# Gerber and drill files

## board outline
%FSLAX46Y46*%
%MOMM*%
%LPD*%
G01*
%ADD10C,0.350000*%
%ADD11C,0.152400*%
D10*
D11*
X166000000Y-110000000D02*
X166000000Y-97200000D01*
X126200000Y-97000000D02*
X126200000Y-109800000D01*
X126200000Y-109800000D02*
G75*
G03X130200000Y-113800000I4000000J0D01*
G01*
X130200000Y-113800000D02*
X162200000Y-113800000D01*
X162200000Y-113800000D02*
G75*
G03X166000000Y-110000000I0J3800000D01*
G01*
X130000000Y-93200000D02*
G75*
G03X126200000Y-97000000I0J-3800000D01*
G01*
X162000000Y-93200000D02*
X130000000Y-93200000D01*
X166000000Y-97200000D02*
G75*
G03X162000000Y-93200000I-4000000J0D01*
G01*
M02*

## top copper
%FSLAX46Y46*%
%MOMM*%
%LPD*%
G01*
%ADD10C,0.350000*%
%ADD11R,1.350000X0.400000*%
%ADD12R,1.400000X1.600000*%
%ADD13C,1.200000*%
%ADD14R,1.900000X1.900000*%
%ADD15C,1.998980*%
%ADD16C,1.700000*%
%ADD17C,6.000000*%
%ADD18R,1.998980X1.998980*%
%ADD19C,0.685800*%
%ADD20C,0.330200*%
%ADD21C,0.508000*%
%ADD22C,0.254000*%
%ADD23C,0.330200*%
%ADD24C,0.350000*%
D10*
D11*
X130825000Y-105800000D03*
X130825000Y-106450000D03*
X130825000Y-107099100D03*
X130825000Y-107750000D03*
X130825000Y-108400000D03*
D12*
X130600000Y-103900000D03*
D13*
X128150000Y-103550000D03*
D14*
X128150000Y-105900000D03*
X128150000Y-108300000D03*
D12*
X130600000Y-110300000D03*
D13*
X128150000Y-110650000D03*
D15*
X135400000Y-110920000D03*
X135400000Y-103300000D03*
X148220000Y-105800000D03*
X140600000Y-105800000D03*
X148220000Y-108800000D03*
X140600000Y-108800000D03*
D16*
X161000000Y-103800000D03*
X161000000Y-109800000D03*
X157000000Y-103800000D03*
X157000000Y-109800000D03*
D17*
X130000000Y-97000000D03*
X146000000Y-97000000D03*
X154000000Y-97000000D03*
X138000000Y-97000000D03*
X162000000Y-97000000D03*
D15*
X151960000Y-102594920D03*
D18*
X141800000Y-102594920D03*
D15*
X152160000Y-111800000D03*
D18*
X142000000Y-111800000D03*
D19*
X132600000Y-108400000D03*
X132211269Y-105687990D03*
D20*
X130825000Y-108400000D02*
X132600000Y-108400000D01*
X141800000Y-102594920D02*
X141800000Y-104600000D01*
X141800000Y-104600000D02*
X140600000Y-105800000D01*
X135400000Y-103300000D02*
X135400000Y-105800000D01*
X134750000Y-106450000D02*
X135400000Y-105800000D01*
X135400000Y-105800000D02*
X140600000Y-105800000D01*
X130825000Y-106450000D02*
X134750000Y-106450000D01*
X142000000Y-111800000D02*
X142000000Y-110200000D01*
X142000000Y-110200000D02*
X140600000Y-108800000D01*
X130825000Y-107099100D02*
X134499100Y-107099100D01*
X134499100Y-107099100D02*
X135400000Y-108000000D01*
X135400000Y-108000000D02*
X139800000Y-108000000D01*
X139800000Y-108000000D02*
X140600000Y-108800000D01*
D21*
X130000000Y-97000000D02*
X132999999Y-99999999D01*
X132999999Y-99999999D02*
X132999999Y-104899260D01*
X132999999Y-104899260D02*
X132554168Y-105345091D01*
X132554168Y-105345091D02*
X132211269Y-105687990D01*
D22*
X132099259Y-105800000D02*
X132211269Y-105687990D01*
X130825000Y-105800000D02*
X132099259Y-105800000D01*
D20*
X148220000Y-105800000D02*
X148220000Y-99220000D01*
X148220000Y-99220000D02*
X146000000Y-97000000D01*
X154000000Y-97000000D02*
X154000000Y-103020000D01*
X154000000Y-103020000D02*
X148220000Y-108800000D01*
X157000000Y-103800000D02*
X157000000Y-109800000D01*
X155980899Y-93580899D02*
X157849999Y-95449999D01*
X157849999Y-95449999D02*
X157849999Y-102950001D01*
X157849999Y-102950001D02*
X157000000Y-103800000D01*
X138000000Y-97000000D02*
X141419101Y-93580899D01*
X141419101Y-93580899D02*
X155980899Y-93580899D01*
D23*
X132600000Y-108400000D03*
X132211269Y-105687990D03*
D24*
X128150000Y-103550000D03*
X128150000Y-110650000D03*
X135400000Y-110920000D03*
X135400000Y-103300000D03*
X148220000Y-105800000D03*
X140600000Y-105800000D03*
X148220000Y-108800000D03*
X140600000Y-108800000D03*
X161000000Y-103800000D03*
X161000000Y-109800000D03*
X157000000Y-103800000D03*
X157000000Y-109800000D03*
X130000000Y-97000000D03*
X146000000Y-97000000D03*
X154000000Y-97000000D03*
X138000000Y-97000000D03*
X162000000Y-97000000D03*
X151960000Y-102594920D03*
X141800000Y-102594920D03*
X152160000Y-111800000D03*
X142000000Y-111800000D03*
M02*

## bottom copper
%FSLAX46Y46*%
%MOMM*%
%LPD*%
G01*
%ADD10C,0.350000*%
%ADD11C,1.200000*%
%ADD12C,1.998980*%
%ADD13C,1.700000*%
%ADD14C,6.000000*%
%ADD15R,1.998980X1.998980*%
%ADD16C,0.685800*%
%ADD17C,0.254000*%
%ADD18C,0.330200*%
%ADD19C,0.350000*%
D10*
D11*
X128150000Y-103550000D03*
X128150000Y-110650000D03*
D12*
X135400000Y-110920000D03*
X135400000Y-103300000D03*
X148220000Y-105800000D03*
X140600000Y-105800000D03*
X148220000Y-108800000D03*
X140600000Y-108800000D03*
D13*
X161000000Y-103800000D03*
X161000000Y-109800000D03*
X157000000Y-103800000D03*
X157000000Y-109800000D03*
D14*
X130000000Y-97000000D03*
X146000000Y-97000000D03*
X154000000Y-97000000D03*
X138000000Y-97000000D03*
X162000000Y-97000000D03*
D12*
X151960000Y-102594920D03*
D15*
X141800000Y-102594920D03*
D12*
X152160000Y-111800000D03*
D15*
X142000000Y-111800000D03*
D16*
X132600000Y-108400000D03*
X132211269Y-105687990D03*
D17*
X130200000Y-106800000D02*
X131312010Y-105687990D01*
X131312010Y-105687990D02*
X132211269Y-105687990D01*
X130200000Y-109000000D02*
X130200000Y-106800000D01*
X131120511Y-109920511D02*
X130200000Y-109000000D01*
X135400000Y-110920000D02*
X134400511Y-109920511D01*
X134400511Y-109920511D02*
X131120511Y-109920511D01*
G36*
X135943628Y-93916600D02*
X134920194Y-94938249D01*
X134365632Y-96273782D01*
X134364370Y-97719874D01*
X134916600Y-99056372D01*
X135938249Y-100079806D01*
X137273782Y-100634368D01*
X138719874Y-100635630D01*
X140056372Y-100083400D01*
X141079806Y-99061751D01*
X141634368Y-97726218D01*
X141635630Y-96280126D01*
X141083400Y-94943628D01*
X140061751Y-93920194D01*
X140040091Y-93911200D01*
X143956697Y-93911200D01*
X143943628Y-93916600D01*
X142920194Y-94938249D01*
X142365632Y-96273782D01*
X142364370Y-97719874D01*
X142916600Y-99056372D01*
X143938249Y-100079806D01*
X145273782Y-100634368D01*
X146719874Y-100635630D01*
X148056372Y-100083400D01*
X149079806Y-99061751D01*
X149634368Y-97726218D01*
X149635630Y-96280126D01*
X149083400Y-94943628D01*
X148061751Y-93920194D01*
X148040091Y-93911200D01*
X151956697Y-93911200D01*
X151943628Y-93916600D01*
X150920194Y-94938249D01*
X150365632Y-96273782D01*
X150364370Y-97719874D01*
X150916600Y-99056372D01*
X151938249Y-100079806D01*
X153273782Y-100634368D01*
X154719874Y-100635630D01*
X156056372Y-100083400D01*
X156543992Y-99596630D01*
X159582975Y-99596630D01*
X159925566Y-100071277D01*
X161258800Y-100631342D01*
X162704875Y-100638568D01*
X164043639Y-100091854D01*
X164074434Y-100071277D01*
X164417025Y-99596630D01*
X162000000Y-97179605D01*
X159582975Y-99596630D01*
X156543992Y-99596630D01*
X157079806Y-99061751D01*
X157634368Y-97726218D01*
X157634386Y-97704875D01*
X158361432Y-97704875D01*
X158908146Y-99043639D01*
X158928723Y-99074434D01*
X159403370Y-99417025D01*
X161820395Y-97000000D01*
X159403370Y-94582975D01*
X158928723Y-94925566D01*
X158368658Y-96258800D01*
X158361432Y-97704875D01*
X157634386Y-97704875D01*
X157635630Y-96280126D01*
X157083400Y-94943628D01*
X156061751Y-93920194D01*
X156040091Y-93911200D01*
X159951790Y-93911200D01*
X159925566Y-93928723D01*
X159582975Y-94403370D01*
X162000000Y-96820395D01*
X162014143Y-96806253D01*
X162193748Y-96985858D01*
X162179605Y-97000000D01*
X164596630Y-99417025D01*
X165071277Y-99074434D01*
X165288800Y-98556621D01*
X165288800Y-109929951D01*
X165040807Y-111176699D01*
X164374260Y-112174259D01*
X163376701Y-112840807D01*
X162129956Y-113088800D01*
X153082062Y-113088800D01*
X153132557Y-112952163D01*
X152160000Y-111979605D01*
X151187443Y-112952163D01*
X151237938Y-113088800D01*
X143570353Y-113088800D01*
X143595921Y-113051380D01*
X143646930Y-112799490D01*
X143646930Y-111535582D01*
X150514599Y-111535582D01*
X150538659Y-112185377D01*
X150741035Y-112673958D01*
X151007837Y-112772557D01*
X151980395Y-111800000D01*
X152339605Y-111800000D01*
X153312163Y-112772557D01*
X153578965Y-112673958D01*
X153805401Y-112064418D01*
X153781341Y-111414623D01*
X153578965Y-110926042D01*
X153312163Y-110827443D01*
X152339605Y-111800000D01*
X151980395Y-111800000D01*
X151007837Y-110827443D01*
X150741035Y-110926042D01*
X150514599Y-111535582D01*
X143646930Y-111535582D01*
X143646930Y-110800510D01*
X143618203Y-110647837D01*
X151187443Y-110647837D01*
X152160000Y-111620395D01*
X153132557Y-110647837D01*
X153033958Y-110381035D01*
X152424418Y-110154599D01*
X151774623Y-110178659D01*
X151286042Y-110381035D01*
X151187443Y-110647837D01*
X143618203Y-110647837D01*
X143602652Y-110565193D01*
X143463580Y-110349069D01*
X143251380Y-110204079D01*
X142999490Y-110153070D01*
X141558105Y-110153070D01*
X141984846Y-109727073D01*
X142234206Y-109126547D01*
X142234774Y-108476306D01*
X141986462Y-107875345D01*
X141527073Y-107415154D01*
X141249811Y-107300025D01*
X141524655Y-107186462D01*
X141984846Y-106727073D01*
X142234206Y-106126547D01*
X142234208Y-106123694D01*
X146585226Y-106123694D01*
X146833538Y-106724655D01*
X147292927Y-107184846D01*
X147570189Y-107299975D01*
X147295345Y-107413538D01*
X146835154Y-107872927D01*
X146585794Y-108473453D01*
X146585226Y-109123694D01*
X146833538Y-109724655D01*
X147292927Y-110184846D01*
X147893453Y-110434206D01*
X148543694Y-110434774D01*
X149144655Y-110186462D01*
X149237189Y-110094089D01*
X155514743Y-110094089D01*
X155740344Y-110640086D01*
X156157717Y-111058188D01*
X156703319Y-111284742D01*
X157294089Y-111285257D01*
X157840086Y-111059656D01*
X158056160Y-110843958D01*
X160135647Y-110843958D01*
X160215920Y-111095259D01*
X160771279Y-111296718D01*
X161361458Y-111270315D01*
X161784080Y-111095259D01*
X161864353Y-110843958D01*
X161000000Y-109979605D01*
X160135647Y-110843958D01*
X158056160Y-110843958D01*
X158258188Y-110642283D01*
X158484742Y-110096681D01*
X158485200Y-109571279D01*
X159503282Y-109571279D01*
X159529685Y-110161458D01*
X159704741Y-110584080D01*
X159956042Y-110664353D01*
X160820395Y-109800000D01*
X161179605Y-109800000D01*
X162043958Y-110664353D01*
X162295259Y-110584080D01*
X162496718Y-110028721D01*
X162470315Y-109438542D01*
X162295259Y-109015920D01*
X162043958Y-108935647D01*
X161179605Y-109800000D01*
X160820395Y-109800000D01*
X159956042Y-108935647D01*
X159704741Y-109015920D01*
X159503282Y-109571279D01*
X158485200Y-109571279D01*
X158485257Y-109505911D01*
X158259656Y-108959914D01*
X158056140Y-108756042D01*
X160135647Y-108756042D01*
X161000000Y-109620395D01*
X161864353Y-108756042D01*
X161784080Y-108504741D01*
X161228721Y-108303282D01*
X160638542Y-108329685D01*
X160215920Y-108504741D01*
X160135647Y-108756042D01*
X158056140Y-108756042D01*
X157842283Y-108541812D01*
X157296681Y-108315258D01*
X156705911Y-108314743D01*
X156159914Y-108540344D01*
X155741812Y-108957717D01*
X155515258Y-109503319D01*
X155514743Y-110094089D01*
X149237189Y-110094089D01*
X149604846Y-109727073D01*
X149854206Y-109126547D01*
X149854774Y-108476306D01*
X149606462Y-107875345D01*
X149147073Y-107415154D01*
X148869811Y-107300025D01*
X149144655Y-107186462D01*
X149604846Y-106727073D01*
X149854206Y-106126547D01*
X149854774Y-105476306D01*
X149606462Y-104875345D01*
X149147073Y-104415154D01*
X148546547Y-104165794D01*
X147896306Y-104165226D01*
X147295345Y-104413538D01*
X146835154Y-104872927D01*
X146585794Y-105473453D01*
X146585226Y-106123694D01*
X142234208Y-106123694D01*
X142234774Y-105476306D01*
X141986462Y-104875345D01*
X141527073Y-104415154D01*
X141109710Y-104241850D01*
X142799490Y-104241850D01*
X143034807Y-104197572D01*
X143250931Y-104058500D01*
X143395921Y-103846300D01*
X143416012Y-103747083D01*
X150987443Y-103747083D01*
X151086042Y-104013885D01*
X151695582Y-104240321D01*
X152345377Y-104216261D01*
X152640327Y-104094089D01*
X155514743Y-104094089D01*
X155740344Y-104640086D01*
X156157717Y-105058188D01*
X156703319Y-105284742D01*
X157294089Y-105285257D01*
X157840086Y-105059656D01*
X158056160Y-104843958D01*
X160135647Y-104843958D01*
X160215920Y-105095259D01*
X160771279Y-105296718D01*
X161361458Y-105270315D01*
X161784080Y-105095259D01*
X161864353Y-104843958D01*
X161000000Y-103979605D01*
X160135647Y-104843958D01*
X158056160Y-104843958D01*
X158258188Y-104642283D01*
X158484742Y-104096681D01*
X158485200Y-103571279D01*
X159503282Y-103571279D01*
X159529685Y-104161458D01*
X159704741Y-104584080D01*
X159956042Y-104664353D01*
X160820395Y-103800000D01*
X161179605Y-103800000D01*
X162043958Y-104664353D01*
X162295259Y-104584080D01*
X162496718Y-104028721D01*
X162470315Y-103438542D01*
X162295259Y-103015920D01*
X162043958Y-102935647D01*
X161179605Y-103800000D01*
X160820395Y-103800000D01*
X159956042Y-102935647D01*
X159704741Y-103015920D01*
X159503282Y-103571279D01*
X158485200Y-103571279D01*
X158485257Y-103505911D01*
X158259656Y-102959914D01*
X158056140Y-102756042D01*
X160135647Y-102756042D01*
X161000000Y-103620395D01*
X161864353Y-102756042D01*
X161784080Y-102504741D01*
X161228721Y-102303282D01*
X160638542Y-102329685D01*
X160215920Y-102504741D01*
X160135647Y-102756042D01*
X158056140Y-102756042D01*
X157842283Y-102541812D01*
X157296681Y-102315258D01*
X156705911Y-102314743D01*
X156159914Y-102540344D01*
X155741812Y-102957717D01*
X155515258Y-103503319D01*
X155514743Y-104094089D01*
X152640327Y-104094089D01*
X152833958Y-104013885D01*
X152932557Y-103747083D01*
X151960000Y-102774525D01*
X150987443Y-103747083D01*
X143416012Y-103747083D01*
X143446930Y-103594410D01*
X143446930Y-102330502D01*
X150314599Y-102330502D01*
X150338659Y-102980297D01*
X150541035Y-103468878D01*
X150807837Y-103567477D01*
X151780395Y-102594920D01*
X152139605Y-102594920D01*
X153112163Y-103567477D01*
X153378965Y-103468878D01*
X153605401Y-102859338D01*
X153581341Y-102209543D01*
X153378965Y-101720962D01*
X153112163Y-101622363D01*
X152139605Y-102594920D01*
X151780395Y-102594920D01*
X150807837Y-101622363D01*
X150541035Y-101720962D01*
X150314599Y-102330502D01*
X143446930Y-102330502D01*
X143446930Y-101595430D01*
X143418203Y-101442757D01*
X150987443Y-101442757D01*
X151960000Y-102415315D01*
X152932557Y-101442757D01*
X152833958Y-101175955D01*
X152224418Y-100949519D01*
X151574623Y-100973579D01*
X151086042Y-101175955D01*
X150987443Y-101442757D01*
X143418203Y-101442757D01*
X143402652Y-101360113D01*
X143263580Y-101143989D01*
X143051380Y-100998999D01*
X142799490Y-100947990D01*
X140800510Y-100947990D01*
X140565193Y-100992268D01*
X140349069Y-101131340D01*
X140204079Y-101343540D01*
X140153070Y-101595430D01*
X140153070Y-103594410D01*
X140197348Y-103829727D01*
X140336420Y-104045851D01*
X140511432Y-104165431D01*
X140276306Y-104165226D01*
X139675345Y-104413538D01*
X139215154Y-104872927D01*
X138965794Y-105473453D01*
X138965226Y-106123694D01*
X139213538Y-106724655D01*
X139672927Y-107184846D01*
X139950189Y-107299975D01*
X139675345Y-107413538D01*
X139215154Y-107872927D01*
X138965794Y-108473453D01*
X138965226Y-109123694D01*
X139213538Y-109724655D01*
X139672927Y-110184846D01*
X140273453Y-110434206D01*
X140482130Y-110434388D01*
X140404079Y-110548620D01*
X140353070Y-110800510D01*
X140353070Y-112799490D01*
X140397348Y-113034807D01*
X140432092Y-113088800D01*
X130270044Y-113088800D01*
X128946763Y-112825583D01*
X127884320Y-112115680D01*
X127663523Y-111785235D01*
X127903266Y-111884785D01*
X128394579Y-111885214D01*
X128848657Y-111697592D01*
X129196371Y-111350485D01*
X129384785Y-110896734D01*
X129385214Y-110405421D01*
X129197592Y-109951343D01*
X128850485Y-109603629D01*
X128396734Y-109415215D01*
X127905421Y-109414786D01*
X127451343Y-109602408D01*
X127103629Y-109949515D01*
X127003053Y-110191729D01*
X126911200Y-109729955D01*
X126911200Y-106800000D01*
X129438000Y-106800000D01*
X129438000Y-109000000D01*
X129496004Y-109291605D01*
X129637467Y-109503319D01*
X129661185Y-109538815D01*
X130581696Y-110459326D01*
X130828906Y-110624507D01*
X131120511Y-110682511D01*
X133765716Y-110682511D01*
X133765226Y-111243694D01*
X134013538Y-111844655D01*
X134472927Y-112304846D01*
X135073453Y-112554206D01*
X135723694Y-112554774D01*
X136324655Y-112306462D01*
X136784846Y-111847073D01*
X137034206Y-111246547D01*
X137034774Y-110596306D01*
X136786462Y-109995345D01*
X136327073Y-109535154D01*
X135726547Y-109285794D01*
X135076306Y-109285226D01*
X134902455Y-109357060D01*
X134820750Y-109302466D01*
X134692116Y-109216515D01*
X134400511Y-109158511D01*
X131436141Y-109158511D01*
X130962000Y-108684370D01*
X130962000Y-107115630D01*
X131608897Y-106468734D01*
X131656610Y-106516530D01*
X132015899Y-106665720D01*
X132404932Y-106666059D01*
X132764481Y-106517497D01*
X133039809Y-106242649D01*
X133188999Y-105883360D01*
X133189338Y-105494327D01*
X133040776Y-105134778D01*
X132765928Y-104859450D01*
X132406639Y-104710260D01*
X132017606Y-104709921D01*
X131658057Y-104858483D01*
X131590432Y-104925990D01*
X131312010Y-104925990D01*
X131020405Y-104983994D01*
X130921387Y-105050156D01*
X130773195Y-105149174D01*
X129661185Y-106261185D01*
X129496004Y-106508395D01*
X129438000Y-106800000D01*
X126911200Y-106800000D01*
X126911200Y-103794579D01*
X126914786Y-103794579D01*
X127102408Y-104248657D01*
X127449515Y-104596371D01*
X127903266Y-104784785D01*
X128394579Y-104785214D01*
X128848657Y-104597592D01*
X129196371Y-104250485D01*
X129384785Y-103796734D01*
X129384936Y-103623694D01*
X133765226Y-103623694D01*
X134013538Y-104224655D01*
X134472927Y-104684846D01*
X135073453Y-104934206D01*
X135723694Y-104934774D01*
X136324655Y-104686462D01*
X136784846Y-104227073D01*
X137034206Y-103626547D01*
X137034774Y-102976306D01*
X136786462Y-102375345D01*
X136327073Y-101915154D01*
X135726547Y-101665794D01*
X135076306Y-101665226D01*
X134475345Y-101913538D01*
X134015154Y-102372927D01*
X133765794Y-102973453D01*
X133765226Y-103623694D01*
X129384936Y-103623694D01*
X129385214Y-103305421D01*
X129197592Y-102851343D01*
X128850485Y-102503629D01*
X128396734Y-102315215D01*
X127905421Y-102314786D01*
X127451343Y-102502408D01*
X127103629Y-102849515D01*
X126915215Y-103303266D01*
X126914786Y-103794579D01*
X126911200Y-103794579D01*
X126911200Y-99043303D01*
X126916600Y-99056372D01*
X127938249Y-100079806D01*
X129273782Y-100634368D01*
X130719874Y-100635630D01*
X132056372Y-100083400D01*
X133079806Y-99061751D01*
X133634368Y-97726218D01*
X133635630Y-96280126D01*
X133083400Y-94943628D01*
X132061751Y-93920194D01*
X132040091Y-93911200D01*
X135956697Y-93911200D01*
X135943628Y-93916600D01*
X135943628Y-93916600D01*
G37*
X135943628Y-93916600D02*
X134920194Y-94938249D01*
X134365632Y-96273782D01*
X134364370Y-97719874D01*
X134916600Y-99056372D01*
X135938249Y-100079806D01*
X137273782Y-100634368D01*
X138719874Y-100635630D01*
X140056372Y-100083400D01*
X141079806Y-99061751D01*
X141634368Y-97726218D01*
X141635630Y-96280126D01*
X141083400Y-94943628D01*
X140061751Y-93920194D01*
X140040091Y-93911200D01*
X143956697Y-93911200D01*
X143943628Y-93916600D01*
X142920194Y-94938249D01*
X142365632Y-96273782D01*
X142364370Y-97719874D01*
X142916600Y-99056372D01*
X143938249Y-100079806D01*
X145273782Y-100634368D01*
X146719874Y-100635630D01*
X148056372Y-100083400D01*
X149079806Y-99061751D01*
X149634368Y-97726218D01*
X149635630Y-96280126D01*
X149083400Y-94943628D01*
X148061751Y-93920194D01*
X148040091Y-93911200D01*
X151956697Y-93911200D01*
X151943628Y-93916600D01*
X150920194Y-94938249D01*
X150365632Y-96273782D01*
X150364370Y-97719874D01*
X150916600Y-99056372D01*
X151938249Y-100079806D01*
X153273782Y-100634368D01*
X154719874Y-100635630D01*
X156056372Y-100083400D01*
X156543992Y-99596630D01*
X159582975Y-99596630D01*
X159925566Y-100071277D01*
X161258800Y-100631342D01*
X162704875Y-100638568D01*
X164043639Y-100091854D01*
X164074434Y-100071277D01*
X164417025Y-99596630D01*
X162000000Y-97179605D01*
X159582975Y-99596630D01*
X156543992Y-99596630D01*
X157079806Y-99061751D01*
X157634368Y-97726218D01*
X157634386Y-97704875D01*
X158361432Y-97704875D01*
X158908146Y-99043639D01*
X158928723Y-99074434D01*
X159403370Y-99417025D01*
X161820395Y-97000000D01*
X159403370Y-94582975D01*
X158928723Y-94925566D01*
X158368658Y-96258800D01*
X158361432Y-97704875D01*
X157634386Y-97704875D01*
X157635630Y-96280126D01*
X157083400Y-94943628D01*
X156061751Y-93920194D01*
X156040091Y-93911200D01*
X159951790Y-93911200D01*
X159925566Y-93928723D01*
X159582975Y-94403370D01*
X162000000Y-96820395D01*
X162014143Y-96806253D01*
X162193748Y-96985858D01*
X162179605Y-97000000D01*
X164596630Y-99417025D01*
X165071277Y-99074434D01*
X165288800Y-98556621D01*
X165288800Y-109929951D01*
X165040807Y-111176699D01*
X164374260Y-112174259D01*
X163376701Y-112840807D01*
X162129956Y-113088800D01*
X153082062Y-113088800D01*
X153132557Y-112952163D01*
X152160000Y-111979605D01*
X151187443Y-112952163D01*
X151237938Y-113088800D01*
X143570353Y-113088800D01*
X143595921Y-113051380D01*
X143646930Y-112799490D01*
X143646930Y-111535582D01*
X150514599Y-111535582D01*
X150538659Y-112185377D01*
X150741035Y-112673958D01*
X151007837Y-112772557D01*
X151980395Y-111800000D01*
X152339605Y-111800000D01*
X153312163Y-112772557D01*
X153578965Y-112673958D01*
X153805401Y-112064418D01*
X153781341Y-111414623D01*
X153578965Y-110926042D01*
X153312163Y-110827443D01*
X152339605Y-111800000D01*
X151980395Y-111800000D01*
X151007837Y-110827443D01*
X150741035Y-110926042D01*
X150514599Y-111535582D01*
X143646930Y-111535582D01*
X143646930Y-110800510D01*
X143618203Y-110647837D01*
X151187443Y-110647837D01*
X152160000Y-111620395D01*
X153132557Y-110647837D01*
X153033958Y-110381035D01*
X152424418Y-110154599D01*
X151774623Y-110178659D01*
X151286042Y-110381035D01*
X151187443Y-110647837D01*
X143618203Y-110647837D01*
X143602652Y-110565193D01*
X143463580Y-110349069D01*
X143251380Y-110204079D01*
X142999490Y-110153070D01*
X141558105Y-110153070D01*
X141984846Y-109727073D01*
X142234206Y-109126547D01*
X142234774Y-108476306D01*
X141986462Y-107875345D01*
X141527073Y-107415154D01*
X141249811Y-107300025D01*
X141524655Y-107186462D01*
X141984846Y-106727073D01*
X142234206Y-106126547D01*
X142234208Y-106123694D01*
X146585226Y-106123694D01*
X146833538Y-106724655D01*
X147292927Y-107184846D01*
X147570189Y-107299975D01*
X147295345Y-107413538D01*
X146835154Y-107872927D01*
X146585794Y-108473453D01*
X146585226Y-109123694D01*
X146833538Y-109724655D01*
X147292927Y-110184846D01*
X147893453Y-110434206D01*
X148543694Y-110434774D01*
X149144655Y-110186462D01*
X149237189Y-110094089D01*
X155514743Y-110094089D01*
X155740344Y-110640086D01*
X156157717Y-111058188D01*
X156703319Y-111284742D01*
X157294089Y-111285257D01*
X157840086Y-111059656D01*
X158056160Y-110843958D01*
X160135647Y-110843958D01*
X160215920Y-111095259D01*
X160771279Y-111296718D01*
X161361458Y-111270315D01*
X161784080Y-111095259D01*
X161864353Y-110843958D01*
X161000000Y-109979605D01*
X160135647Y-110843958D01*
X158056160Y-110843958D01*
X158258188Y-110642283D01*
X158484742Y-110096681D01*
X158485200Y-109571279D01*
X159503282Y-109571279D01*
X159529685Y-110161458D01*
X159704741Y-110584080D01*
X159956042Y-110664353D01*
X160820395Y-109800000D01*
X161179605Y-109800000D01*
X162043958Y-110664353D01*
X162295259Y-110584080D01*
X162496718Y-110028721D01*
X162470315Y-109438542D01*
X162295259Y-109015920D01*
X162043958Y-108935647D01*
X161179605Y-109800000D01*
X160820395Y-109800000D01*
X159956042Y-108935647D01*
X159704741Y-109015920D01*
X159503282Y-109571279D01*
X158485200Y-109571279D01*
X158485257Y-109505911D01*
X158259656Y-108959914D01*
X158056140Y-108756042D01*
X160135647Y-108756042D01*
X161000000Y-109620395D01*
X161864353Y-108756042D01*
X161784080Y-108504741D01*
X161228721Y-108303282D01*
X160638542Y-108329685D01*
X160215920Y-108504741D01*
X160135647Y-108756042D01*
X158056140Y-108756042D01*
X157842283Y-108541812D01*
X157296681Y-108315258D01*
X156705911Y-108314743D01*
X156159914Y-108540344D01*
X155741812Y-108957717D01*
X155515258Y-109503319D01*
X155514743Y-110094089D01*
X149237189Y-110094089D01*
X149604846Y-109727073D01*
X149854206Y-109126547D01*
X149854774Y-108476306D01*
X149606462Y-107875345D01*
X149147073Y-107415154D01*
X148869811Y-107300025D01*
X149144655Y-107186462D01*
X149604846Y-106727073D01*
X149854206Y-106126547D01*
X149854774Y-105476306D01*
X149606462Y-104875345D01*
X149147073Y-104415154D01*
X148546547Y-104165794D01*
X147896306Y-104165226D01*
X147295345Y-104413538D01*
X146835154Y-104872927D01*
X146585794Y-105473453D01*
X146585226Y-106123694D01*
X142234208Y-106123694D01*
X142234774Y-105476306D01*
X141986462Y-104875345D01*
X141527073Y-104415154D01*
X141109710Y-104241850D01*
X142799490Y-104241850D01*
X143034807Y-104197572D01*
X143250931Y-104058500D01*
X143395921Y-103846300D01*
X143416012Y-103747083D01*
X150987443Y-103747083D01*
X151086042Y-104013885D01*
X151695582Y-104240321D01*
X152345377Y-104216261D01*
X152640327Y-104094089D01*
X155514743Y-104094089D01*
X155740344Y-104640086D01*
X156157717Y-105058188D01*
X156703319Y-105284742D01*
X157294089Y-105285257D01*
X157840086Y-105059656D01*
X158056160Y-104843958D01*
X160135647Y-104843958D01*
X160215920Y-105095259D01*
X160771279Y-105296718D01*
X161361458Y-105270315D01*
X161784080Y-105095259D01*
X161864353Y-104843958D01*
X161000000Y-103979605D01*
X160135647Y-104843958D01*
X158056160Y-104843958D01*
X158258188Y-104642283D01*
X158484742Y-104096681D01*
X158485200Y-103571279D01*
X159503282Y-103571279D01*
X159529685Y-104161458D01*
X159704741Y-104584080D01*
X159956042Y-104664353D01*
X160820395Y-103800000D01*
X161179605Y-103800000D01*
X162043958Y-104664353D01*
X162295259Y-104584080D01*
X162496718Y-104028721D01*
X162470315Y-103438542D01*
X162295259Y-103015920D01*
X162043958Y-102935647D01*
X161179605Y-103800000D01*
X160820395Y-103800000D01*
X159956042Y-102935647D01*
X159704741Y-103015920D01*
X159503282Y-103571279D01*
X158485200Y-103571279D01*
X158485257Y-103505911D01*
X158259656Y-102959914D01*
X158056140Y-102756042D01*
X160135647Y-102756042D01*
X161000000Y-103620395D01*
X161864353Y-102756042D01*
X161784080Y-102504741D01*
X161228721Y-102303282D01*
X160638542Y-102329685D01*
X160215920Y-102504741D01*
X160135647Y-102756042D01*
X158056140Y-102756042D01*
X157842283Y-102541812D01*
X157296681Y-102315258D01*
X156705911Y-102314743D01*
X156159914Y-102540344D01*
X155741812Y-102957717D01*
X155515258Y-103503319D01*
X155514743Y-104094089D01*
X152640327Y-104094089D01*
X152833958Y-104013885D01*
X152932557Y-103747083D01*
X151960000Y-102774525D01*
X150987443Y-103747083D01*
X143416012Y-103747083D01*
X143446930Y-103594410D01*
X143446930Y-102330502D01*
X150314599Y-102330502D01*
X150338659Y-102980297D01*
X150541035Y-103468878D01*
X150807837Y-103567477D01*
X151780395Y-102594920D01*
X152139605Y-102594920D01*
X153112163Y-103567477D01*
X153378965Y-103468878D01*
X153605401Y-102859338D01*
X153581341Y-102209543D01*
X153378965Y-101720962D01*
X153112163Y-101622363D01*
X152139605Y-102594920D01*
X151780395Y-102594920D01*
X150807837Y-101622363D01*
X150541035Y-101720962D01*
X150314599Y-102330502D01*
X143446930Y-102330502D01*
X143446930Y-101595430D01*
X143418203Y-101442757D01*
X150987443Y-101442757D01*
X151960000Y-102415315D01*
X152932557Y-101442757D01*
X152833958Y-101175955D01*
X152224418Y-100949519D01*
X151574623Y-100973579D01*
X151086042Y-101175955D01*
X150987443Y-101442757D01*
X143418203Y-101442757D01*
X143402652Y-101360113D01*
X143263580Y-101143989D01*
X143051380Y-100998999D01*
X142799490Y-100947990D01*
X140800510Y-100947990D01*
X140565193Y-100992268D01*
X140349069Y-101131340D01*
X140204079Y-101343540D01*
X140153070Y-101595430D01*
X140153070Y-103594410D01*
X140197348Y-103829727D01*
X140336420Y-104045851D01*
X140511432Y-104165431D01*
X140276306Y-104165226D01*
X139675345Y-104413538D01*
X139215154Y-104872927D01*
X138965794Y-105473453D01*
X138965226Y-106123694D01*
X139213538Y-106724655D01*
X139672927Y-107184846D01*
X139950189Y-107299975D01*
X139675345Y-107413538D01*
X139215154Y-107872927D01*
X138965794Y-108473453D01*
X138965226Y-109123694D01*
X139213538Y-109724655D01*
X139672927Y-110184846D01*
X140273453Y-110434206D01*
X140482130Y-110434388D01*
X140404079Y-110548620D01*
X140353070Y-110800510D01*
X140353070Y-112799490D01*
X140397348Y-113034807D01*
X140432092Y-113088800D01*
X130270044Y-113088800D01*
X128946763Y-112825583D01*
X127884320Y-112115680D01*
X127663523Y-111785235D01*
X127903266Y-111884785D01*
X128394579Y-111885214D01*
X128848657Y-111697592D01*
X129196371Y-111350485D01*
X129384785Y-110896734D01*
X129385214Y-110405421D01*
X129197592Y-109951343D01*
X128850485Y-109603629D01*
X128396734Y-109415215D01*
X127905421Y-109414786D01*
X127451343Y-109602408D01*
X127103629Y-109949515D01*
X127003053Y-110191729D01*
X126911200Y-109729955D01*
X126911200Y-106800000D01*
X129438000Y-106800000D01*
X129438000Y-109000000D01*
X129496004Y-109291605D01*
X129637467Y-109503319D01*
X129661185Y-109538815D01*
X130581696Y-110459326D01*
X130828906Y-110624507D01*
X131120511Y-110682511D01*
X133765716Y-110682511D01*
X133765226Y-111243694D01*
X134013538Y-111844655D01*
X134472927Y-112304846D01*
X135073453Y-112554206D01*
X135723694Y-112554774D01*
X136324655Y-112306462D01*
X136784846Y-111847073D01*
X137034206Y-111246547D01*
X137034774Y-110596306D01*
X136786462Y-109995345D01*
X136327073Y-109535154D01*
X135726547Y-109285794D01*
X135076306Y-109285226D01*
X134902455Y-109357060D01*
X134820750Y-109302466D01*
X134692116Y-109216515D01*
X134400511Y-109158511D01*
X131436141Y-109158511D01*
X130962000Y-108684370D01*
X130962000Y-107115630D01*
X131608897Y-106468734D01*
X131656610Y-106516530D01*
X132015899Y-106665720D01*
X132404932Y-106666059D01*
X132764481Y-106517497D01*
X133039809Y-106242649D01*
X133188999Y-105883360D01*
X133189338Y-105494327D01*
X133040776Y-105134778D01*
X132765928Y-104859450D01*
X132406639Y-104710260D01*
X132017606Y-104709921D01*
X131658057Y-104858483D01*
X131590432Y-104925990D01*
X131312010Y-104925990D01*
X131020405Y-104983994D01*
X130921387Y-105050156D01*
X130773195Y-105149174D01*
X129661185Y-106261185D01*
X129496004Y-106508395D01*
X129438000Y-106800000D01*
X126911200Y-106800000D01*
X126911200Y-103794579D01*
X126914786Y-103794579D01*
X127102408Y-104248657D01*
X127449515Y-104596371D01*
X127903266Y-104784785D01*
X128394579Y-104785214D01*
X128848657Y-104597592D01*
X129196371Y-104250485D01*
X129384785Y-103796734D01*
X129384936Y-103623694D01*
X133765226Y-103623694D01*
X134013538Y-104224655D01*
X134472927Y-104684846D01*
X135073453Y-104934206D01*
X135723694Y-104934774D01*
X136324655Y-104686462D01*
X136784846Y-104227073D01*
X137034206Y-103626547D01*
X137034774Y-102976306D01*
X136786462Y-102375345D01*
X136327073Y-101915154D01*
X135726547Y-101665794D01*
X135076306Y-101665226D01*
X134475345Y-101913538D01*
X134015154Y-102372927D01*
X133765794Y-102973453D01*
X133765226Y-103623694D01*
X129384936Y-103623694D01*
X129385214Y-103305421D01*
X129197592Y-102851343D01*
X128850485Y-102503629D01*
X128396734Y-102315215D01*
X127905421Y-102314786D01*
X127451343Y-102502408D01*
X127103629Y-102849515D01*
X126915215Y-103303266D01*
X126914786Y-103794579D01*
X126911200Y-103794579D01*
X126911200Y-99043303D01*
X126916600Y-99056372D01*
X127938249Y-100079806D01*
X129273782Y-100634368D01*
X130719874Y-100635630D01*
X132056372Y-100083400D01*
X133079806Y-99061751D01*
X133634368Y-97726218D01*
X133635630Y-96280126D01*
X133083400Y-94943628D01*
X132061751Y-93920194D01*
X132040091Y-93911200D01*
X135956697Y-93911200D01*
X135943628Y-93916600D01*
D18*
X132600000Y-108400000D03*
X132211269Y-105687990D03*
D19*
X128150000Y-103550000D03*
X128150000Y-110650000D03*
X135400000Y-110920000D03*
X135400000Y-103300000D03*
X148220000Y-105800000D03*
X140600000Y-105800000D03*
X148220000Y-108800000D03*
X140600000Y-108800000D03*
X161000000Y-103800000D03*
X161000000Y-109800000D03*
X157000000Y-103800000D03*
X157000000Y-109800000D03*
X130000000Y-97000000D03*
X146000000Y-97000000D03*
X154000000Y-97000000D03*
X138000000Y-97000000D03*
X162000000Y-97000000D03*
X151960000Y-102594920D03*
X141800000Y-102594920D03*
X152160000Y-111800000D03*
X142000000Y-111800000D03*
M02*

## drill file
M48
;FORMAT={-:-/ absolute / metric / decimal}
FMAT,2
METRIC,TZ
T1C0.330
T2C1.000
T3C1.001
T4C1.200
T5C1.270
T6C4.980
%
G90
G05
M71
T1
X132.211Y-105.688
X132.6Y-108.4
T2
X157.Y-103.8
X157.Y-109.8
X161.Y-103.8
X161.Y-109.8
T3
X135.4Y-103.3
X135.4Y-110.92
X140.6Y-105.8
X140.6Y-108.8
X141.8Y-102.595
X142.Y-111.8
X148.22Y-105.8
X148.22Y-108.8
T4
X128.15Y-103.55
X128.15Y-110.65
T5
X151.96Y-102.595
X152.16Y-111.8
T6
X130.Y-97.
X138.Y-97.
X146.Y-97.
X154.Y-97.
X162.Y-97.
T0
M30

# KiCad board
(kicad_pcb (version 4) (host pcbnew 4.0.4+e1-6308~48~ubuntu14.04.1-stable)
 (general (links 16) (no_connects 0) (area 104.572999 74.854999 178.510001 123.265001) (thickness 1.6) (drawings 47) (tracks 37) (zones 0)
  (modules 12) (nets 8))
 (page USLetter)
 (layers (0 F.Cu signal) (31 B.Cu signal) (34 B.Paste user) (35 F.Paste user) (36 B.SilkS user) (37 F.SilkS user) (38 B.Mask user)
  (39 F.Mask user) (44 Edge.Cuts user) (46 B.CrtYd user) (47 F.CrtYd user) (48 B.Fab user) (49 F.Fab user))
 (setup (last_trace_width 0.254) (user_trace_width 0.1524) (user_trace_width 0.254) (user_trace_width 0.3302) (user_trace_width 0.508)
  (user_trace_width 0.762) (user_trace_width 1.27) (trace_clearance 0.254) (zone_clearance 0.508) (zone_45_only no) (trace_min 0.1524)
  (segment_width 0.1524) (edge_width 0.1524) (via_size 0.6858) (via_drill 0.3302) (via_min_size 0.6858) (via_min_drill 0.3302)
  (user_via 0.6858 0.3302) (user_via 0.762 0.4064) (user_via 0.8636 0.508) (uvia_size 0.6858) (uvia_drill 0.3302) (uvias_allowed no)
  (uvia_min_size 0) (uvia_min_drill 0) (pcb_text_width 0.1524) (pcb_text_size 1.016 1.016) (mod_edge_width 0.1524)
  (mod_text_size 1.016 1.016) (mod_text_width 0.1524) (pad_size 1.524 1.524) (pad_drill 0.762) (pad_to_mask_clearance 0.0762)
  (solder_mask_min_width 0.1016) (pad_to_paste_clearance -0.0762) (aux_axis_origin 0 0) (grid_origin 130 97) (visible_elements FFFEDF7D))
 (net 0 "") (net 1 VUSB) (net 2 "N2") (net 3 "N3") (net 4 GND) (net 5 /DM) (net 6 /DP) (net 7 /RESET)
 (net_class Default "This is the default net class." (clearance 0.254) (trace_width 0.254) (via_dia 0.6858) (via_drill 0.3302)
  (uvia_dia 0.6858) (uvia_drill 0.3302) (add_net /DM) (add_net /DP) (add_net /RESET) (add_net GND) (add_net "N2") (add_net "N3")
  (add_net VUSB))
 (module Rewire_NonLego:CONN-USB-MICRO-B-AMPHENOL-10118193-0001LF (layer F.Cu) (at 128.15 107.1 270)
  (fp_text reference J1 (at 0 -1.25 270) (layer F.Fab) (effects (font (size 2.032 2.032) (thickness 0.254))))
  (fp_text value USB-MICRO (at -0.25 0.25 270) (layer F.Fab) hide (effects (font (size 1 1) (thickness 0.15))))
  (pad 1 smd rect (at -1.3 -2.675) (size 1.35 0.4) (layers F.Cu F.Paste F.Mask) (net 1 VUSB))
  (pad 2 smd rect (at -0.65 -2.675) (size 1.35 0.4) (layers F.Cu F.Paste F.Mask) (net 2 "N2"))
  (pad 3 smd rect (at -0.0009 -2.675) (size 1.35 0.4) (layers F.Cu F.Paste F.Mask) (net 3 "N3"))
  (pad 4 smd rect (at 0.65 -2.675) (size 1.35 0.4) (layers F.Cu F.Paste F.Mask))
  (pad 5 smd rect (at 1.3 -2.675) (size 1.35 0.4) (layers F.Cu F.Paste F.Mask) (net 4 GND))
  (pad 6 smd rect (at -3.2 -2.45) (size 1.4 1.6) (layers F.Cu F.Paste F.Mask))
  (pad 6 thru_hole circle (at -3.55 0) (size 1.2 1.2) (drill 1.2) (layers *.Cu *.Mask F.SilkS))
  (pad 6 smd rect (at -1.2 0) (size 1.9 1.9) (layers F.Cu F.Paste F.Mask))
  (pad 6 smd rect (at 1.2 0) (size 1.9 1.9) (layers F.Cu F.Paste F.Mask))
  (pad 6 smd rect (at 3.2 -2.45) (size 1.4 1.6) (layers F.Cu F.Paste F.Mask))
  (pad 6 thru_hole circle (at 3.55 0) (size 1.2 1.2) (drill 1.2) (layers *.Cu *.Mask F.SilkS)))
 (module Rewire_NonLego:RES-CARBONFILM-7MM (layer F.Cu) (at 135.4 110.92 90)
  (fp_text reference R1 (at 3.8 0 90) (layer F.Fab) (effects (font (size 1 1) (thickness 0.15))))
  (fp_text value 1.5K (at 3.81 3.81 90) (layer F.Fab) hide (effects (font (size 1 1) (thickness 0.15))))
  (pad 1 thru_hole circle (at 0 0 90) (size 1.99898 1.99898) (drill 1.00076) (layers *.Cu *.SilkS *.Mask) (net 1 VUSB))
  (pad 2 thru_hole circle (at 7.62 0 90) (size 1.99898 1.99898) (drill 1.00076) (layers *.Cu *.SilkS *.Mask) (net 2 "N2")))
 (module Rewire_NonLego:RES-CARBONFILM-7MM (layer F.Cu) (at 148.22 105.8 180)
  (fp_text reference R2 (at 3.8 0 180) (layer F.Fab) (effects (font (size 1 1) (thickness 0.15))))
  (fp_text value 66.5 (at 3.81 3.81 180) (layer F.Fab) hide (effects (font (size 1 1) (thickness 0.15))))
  (pad 1 thru_hole circle (at 0 0 180) (size 1.99898 1.99898) (drill 1.00076) (layers *.Cu *.SilkS *.Mask) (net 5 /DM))
  (pad 2 thru_hole circle (at 7.62 0 180) (size 1.99898 1.99898) (drill 1.00076) (layers *.Cu *.SilkS *.Mask) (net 2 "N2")))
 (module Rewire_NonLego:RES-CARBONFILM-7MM (layer F.Cu) (at 148.22 108.8 180)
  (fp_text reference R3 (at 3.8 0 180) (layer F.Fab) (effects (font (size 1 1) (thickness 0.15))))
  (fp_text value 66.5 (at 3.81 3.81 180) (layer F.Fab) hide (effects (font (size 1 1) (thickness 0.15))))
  (pad 1 thru_hole circle (at 0 0 180) (size 1.99898 1.99898) (drill 1.00076) (layers *.Cu *.SilkS *.Mask) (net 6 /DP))
  (pad 2 thru_hole circle (at 7.62 0 180) (size 1.99898 1.99898) (drill 1.00076) (layers *.Cu *.SilkS *.Mask) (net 3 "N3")))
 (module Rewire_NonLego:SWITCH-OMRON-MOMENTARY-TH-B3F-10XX (layer F.Cu) (at 157 109.8 90)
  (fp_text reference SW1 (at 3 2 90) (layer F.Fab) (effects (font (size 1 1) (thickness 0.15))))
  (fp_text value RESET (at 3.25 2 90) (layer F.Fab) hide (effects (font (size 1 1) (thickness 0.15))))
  (pad 4 thru_hole circle (at 6 4 90) (size 1.7 1.7) (drill 1) (layers *.Cu *.Mask) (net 4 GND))
  (pad 3 thru_hole circle (at 0 4 90) (size 1.7 1.7) (drill 1) (layers *.Cu *.Mask) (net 4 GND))
  (pad 2 thru_hole circle (at 6 0 90) (size 1.7 1.7) (drill 1) (layers *.Cu *.Mask) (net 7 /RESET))
  (pad 1 thru_hole circle (at 0 0 90) (size 1.7 1.7) (drill 1) (layers *.Cu *.Mask) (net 7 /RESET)))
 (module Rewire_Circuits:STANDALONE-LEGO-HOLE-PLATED (layer F.Cu) (at 130 97)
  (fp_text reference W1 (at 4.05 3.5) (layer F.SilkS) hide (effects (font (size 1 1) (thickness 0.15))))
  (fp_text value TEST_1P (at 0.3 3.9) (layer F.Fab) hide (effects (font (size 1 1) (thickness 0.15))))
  (pad 1 thru_hole circle (at 0 0) (size 6 6) (drill 4.98) (layers *.Cu *.Mask) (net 1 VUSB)))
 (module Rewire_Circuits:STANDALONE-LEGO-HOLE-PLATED (layer F.Cu) (at 146 97)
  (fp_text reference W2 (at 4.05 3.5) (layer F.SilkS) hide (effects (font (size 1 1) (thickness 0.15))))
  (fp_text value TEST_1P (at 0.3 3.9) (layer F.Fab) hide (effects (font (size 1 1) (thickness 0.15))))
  (pad 1 thru_hole circle (at 0 0) (size 6 6) (drill 4.98) (layers *.Cu *.Mask) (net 5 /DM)))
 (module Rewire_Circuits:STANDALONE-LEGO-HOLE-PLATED (layer F.Cu) (at 154 97)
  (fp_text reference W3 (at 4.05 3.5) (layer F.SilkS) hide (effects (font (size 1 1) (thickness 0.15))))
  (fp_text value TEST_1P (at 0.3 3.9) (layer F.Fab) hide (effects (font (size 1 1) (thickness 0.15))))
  (pad 1 thru_hole circle (at 0 0) (size 6 6) (drill 4.98) (layers *.Cu *.Mask) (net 6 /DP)))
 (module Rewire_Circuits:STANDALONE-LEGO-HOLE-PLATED (layer F.Cu) (at 138 97)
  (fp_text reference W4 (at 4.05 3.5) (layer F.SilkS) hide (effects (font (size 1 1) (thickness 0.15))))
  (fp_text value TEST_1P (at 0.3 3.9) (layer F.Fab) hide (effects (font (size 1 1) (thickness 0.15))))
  (pad 1 thru_hole circle (at 0 0) (size 6 6) (drill 4.98) (layers *.Cu *.Mask) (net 7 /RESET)))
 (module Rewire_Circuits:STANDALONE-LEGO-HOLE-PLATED (layer F.Cu) (at 162 97)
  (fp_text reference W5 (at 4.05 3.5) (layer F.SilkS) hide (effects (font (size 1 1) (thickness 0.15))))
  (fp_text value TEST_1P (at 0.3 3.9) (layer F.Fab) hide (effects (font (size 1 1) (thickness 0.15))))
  (pad 1 thru_hole circle (at 0 0) (size 6 6) (drill 4.98) (layers *.Cu *.Mask) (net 4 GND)))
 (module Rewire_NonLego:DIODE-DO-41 (layer F.Cu) (at 141.8 102.59746)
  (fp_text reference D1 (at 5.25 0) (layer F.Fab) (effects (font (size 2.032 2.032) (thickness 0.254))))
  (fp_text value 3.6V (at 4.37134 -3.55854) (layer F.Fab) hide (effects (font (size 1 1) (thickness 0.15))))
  (pad 2 thru_hole circle (at 10.16 -0.00254 180) (size 1.99898 1.99898) (drill 1.27) (layers *.Cu *.Mask F.SilkS) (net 4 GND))
  (pad 1 thru_hole rect (at 0 -0.00254 180) (size 1.99898 1.99898) (drill 1.00076) (layers *.Cu *.Mask F.SilkS) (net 2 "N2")))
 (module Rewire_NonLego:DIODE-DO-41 (layer F.Cu) (at 142 111.80254)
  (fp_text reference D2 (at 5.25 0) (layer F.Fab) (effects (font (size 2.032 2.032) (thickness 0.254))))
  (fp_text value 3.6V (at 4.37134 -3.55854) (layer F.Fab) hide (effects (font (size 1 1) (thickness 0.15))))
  (pad 2 thru_hole circle (at 10.16 -0.00254 180) (size 1.99898 1.99898) (drill 1.27) (layers *.Cu *.Mask F.SilkS) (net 4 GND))
  (pad 1 thru_hole rect (at 0 -0.00254 180) (size 1.99898 1.99898) (drill 1.00076) (layers *.Cu *.Mask F.SilkS) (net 3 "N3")))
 (gr_line (start 166 110) (end 166 97.2) (layer Edge.Cuts) (width 0.1524))
 (gr_line (start 126.2 97) (end 126.2 109.8) (layer Edge.Cuts) (width 0.1524))
 (gr_arc (start 130.2 109.8) (end 130.2 113.8) (angle 90) (layer Edge.Cuts) (width 0.1524))
 (gr_line (start 130.2 113.8) (end 162.2 113.8) (layer Edge.Cuts) (width 0.1524))
 (gr_arc (start 162.2 110) (end 166 110) (angle 90) (layer Edge.Cuts) (width 0.1524))
 (gr_arc (start 130 97) (end 126.2 97) (angle 90) (layer Edge.Cuts) (width 0.1524))
 (gr_line (start 162 93.2) (end 130 93.2) (layer Edge.Cuts) (width 0.1524))
 (gr_arc (start 162 97.2) (end 162 93.2) (angle 90) (layer Edge.Cuts) (width 0.1524))
 (segment (start 130.825 108.4) (end 132.6 108.4) (width 0.3302) (layer F.Cu) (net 4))
 (via (at 132.6 108.4) (size 0.6858) (drill 0.3302) (layers F.Cu B.Cu) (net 4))
 (segment (start 141.8 102.59492) (end 141.8 104.6) (width 0.3302) (layer F.Cu) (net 2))
 (segment (start 141.8 104.6) (end 140.6 105.8) (width 0.3302) (layer F.Cu) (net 2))
 (segment (start 135.4 103.3) (end 135.4 105.8) (width 0.3302) (layer F.Cu) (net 2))
 (segment (start 134.75 106.45) (end 135.4 105.8) (width 0.3302) (layer F.Cu) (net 2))
 (segment (start 135.4 105.8) (end 140.6 105.8) (width 0.3302) (layer F.Cu) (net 2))
 (segment (start 130.825 106.45) (end 134.75 106.45) (width 0.3302) (layer F.Cu) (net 2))
 (segment (start 142 111.8) (end 142 110.2) (width 0.3302) (layer F.Cu) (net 3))
 (segment (start 142 110.2) (end 140.6 108.8) (width 0.3302) (layer F.Cu) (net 3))
 (segment (start 130.825 107.0991) (end 134.4991 107.0991) (width 0.3302) (layer F.Cu) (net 3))
 (segment (start 134.4991 107.0991) (end 135.4 108) (width 0.3302) (layer F.Cu) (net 3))
 (segment (start 135.4 108) (end 139.8 108) (width 0.3302) (layer F.Cu) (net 3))
 (segment (start 139.8 108) (end 140.6 108.8) (width 0.3302) (layer F.Cu) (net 3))
 (segment (start 130.2 106.8) (end 131.31201 105.68799) (width 0.254) (layer B.Cu) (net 1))
 (segment (start 131.31201 105.68799) (end 132.211269 105.68799) (width 0.254) (layer B.Cu) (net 1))
 (segment (start 130.2 109) (end 130.2 106.8) (width 0.254) (layer B.Cu) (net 1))
 (segment (start 131.120511 109.920511) (end 130.2 109) (width 0.254) (layer B.Cu) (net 1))
 (segment (start 135.4 110.92) (end 134.400511 109.920511) (width 0.254) (layer B.Cu) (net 1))
 (segment (start 134.400511 109.920511) (end 131.120511 109.920511) (width 0.254) (layer B.Cu) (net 1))
 (segment (start 130 97) (end 132.999999 99.999999) (width 0.508) (layer F.Cu) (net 1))
 (segment (start 132.999999 99.999999) (end 132.999999 104.89926) (width 0.508) (layer F.Cu) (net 1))
 (segment (start 132.999999 104.89926) (end 132.554168 105.345091) (width 0.508) (layer F.Cu) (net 1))
 (segment (start 132.554168 105.345091) (end 132.211269 105.68799) (width 0.508) (layer F.Cu) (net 1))
 (segment (start 132.099259 105.8) (end 132.211269 105.68799) (width 0.254) (layer F.Cu) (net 1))
 (segment (start 130.825 105.8) (end 132.099259 105.8) (width 0.254) (layer F.Cu) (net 1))
 (via (at 132.211269 105.68799) (size 0.6858) (drill 0.3302) (layers F.Cu B.Cu) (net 1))
 (segment (start 148.22 105.8) (end 148.22 99.22) (width 0.3302) (layer F.Cu) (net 5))
 (segment (start 148.22 99.22) (end 146 97) (width 0.3302) (layer F.Cu) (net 5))
 (segment (start 154 97) (end 154 103.02) (width 0.3302) (layer F.Cu) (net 6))
 (segment (start 154 103.02) (end 148.22 108.8) (width 0.3302) (layer F.Cu) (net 6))
 (segment (start 157 103.8) (end 157 109.8) (width 0.3302) (layer F.Cu) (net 7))
 (segment (start 155.980899 93.580899) (end 157.849999 95.449999) (width 0.3302) (layer F.Cu) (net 7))
 (segment (start 157.849999 95.449999) (end 157.849999 102.950001) (width 0.3302) (layer F.Cu) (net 7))
 (segment (start 157.849999 102.950001) (end 157 103.8) (width 0.3302) (layer F.Cu) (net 7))
 (segment (start 138 97) (end 141.419101 93.580899) (width 0.3302) (layer F.Cu) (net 7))
 (segment (start 141.419101 93.580899) (end 155.980899 93.580899) (width 0.3302) (layer F.Cu) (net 7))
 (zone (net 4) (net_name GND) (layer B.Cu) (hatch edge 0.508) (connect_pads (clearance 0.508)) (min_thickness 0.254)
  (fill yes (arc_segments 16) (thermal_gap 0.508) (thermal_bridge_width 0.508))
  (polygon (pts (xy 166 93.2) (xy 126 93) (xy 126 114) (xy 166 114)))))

